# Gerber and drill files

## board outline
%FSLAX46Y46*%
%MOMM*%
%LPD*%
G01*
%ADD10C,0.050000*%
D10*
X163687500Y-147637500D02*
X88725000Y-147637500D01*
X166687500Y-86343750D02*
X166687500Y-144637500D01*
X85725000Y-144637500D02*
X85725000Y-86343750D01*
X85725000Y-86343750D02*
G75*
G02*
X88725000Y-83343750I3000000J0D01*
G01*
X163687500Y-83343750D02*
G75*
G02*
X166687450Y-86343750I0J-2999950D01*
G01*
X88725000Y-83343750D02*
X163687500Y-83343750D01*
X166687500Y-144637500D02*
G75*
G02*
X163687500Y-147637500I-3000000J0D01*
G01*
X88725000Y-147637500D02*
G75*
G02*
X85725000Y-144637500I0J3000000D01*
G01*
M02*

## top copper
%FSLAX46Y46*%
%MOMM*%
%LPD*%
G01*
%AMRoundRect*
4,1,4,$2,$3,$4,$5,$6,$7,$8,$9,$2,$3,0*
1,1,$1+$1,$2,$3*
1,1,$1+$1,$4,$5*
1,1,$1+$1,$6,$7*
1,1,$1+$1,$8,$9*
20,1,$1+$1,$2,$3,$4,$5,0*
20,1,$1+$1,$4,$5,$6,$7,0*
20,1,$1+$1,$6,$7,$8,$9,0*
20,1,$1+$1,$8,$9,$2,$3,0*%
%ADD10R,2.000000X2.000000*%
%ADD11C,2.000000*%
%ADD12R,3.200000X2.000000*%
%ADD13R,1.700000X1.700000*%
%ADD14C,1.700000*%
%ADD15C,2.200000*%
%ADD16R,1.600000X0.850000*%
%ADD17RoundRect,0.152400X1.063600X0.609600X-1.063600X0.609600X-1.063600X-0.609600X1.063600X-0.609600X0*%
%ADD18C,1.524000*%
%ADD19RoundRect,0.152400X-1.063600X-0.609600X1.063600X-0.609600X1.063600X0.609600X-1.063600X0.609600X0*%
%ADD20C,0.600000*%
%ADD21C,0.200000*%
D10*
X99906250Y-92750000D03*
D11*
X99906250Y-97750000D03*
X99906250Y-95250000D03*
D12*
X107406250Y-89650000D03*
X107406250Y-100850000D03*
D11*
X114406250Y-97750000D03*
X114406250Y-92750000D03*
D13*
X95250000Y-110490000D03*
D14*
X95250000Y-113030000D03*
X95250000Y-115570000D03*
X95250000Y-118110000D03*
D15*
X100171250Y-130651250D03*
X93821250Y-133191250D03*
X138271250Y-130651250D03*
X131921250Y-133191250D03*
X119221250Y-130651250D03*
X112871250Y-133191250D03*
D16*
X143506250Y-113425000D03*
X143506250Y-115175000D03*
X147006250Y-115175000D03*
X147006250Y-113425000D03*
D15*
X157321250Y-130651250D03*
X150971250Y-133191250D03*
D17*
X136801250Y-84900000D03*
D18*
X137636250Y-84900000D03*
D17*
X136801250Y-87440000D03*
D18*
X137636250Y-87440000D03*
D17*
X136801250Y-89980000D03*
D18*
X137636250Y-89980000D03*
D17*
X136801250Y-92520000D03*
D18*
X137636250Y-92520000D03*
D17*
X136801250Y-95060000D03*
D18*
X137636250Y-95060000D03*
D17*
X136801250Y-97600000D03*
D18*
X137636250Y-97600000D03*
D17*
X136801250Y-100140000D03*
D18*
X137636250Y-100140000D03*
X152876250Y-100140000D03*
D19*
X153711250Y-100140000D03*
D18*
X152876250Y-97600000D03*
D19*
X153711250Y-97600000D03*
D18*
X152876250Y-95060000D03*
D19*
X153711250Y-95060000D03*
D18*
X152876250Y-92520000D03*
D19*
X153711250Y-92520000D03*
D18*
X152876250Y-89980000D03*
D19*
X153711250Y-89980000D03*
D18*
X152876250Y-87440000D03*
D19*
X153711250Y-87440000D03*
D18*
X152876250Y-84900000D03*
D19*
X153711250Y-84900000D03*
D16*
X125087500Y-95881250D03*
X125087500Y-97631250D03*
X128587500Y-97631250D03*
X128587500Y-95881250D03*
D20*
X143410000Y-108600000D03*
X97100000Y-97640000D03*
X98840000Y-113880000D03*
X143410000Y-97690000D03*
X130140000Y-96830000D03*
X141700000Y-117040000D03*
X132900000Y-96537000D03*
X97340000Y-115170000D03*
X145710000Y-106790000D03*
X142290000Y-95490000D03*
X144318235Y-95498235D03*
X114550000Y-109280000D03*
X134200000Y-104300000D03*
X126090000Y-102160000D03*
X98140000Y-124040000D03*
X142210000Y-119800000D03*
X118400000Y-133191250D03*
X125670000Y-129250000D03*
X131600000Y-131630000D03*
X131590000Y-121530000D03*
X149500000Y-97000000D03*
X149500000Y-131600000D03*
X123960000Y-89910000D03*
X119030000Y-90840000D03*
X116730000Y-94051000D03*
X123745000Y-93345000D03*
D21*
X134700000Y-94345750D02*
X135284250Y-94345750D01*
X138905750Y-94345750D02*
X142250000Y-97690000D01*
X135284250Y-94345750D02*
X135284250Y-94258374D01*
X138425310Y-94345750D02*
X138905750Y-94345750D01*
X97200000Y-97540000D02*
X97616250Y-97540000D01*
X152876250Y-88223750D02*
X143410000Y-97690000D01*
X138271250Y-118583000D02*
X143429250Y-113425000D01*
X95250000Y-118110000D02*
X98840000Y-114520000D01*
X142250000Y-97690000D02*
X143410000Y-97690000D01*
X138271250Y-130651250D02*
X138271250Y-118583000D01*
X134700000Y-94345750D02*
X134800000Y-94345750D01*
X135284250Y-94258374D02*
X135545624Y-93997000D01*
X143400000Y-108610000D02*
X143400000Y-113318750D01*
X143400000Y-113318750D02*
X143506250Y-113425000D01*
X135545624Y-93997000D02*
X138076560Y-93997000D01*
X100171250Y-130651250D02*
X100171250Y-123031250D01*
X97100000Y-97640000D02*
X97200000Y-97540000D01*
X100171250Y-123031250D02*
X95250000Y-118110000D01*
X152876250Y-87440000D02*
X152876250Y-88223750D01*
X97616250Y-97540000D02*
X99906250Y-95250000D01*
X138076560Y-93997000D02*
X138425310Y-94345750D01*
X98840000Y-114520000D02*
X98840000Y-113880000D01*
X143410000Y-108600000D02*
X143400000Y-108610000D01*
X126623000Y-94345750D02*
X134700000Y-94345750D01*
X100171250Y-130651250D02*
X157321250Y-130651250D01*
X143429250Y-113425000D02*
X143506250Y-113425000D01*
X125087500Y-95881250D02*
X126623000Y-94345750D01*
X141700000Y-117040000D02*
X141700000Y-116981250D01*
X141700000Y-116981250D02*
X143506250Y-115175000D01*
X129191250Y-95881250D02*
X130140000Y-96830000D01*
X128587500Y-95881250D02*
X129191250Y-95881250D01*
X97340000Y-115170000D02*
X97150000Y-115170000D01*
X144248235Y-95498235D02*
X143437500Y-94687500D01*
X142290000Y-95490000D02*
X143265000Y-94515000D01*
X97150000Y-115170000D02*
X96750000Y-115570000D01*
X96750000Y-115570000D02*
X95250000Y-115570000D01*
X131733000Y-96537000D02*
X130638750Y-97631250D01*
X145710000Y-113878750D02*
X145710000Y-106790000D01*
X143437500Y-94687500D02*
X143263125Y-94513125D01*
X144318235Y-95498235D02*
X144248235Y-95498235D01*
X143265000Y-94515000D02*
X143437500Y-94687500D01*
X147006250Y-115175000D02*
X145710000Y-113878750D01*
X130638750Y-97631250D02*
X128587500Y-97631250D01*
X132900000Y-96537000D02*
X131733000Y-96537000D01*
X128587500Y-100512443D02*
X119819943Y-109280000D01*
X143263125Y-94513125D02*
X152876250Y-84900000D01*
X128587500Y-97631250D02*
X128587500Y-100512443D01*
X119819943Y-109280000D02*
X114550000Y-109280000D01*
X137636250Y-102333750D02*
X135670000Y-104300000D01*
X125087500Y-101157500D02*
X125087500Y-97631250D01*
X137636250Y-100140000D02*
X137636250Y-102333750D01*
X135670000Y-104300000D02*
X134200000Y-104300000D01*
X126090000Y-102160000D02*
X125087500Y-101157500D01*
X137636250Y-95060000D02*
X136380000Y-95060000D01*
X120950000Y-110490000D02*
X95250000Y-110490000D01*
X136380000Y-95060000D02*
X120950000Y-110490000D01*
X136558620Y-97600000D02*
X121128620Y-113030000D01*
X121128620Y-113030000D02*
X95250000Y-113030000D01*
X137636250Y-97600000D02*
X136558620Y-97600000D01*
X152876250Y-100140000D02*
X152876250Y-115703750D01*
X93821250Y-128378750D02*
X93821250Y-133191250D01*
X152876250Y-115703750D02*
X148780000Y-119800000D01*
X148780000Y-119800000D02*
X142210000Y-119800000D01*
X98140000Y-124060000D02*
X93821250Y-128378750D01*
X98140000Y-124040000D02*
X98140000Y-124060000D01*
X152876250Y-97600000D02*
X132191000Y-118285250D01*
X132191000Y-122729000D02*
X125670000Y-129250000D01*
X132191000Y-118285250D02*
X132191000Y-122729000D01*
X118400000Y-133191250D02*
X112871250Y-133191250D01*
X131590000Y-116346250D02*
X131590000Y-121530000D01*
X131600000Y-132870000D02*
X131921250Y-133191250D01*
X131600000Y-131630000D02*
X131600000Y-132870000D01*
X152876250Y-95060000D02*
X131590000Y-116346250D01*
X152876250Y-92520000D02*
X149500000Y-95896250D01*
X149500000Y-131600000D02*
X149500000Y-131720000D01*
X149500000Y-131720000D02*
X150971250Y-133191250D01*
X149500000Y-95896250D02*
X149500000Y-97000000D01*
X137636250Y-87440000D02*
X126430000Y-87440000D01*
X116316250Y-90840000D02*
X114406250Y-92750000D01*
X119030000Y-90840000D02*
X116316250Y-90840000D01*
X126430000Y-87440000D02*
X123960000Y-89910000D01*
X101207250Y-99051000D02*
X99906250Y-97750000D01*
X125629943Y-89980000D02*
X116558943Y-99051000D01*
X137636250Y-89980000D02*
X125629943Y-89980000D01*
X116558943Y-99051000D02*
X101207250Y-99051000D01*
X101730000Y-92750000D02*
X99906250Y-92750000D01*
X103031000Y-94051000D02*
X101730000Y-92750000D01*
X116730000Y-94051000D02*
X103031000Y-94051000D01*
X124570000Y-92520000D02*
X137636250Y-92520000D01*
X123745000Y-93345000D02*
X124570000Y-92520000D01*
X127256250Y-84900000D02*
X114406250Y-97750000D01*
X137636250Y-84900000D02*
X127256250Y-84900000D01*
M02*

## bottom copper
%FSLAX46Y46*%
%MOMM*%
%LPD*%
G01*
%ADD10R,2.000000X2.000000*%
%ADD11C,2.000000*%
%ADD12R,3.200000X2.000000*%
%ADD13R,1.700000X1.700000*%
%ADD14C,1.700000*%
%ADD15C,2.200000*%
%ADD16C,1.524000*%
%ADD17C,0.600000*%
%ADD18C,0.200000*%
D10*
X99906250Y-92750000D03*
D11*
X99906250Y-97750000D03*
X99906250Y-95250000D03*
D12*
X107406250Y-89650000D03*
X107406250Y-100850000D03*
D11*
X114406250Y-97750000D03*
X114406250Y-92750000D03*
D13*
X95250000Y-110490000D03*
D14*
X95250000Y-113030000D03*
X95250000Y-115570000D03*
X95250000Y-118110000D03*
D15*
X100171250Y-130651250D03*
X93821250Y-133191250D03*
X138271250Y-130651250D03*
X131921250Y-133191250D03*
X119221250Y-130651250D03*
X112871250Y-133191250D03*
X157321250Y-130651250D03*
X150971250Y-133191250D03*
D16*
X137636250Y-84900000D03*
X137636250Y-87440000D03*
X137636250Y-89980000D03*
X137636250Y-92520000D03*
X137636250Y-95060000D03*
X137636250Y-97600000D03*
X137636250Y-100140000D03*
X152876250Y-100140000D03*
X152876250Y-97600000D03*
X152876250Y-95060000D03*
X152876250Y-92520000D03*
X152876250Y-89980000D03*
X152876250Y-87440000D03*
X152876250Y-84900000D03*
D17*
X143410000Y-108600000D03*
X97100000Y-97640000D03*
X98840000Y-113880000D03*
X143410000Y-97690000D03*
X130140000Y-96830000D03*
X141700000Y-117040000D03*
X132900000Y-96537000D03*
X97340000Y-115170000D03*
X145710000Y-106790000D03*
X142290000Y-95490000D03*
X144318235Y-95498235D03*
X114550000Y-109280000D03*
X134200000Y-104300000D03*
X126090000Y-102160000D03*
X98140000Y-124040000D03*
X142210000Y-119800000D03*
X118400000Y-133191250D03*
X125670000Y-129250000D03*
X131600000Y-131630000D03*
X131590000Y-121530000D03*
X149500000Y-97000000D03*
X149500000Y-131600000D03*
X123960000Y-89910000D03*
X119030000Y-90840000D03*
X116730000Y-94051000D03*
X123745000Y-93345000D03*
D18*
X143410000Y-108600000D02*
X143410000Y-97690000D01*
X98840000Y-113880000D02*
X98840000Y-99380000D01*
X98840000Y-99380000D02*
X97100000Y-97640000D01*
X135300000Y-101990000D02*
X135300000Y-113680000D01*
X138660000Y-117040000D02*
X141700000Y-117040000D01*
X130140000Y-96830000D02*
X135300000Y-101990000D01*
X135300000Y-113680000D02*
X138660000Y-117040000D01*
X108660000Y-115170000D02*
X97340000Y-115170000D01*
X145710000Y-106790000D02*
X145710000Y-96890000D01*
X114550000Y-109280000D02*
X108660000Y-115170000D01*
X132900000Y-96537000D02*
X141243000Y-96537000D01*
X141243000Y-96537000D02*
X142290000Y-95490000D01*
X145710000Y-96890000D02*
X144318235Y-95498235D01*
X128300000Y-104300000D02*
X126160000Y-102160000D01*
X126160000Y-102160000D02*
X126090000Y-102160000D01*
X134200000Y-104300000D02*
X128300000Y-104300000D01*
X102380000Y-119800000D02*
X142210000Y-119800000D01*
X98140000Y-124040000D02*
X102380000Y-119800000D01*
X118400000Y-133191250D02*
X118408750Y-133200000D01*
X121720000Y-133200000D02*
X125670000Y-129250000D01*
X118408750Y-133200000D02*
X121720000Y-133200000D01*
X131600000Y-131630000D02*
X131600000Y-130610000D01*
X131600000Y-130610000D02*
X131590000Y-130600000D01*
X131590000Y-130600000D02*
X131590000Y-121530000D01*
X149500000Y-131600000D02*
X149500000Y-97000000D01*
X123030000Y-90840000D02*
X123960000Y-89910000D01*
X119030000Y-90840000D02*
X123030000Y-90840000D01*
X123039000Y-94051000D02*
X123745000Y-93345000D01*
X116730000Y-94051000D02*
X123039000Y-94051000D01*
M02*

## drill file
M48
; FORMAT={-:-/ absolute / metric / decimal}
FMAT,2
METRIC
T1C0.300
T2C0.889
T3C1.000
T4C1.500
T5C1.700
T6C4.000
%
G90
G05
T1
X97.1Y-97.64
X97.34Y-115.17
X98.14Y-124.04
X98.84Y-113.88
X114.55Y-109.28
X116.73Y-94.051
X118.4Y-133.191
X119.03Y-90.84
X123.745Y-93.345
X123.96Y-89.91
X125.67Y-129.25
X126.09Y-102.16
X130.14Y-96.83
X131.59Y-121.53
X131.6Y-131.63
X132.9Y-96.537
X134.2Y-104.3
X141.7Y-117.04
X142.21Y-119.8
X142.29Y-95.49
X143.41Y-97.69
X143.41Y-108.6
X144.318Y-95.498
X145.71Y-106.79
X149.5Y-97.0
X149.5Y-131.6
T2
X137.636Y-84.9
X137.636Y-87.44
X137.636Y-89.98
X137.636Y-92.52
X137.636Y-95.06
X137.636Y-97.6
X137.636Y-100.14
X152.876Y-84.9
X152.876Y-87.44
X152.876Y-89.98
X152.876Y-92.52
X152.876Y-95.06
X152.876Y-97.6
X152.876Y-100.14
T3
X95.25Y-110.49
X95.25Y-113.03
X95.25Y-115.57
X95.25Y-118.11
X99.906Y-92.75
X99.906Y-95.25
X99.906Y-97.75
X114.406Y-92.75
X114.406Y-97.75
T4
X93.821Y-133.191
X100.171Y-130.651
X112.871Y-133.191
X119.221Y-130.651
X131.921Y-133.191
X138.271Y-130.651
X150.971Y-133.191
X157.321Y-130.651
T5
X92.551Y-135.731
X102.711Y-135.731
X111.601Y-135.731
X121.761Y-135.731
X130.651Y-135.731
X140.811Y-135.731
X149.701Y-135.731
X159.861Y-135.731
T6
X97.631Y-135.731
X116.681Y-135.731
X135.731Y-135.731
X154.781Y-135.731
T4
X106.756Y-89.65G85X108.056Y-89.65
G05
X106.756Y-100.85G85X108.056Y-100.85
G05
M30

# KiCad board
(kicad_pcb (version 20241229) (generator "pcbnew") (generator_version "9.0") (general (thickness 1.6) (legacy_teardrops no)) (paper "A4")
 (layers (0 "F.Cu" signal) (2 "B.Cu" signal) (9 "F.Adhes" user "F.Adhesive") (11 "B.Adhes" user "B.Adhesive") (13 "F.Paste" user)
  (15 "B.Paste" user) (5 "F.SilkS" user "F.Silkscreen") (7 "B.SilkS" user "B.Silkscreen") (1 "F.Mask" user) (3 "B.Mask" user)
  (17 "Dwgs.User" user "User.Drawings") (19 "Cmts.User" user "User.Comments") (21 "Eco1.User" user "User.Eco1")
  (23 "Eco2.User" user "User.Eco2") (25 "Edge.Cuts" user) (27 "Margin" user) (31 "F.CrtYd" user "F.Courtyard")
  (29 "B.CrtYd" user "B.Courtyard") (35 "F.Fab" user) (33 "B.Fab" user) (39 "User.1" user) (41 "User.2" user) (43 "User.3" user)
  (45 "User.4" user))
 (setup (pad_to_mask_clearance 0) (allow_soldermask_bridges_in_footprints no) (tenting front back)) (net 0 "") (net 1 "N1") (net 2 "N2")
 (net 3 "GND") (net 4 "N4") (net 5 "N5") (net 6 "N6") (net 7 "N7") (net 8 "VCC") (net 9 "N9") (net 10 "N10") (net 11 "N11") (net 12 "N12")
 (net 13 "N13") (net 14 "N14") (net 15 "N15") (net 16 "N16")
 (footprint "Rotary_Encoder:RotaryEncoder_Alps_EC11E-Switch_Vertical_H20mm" (layer "F.Cu") (at 99.90625 92.75)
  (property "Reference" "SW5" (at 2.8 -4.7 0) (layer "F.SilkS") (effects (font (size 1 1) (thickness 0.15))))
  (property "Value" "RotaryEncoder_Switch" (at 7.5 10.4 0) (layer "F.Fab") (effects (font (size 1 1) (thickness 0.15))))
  (pad "A" thru_hole rect (at 0 0) (size 2 2) (drill 1) (layers "*.Cu" "*.Mask") (remove_unused_layers no) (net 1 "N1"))
  (pad "B" thru_hole circle (at 0 5) (size 2 2) (drill 1) (layers "*.Cu" "*.Mask") (remove_unused_layers no) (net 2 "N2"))
  (pad "C" thru_hole circle (at 0 2.5) (size 2 2) (drill 1) (layers "*.Cu" "*.Mask") (remove_unused_layers no) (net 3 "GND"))
  (pad "MP" thru_hole rect (at 7.5 -3.1) (size 3.2 2) (drill oval 2.8 1.5) (layers "*.Cu" "*.Mask") (remove_unused_layers no))
  (pad "MP" thru_hole rect (at 7.5 8.1) (size 3.2 2) (drill oval 2.8 1.5) (layers "*.Cu" "*.Mask") (remove_unused_layers no))
  (pad "S1" thru_hole circle (at 14.5 5) (size 2 2) (drill 1) (layers "*.Cu" "*.Mask") (remove_unused_layers no) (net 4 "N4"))
  (pad "S2" thru_hole circle (at 14.5 0) (size 2 2) (drill 1) (layers "*.Cu" "*.Mask") (remove_unused_layers no) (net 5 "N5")))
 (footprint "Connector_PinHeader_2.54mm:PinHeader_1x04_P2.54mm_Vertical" (layer "F.Cu") (at 95.25 110.49)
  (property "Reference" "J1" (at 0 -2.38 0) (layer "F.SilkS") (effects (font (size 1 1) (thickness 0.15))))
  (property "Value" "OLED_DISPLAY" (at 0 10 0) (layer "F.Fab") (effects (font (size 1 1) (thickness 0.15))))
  (pad "1" thru_hole rect (at 0 0) (size 1.7 1.7) (drill 1) (layers "*.Cu" "*.Mask") (remove_unused_layers no) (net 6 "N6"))
  (pad "2" thru_hole circle (at 0 2.54) (size 1.7 1.7) (drill 1) (layers "*.Cu" "*.Mask") (remove_unused_layers no) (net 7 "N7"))
  (pad "3" thru_hole circle (at 0 5.08) (size 1.7 1.7) (drill 1) (layers "*.Cu" "*.Mask") (remove_unused_layers no) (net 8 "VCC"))
  (pad "4" thru_hole circle (at 0 7.62) (size 1.7 1.7) (drill 1) (layers "*.Cu" "*.Mask") (remove_unused_layers no) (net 3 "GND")))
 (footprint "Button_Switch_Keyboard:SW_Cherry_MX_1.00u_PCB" (layer "F.Cu") (at 100.17125 130.65125)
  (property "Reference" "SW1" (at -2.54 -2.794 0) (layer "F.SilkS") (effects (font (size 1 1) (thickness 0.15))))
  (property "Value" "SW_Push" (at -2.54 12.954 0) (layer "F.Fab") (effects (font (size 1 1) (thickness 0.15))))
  (pad "" np_thru_hole circle (at -7.62 5.08) (size 1.7 1.7) (drill 1.7) (layers "*.Cu" "*.Mask"))
  (pad "" np_thru_hole circle (at -2.54 5.08) (size 4 4) (drill 4) (layers "*.Cu" "*.Mask"))
  (pad "" np_thru_hole circle (at 2.54 5.08) (size 1.7 1.7) (drill 1.7) (layers "*.Cu" "*.Mask"))
  (pad "1" thru_hole circle (at 0 0) (size 2.2 2.2) (drill 1.5) (layers "*.Cu" "*.Mask") (remove_unused_layers no) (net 3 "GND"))
  (pad "2" thru_hole circle (at -6.35 2.54) (size 2.2 2.2) (drill 1.5) (layers "*.Cu" "*.Mask") (remove_unused_layers no) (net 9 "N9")))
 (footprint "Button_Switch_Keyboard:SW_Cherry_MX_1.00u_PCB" (layer "F.Cu") (at 138.27125 130.65125)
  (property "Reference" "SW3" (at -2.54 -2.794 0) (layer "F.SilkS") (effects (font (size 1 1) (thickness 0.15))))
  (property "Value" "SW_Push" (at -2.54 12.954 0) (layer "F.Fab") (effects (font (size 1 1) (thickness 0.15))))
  (pad "" np_thru_hole circle (at -7.62 5.08) (size 1.7 1.7) (drill 1.7) (layers "*.Cu" "*.Mask"))
  (pad "" np_thru_hole circle (at -2.54 5.08) (size 4 4) (drill 4) (layers "*.Cu" "*.Mask"))
  (pad "" np_thru_hole circle (at 2.54 5.08) (size 1.7 1.7) (drill 1.7) (layers "*.Cu" "*.Mask"))
  (pad "1" thru_hole circle (at 0 0) (size 2.2 2.2) (drill 1.5) (layers "*.Cu" "*.Mask") (remove_unused_layers no) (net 3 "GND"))
  (pad "2" thru_hole circle (at -6.35 2.54) (size 2.2 2.2) (drill 1.5) (layers "*.Cu" "*.Mask") (remove_unused_layers no) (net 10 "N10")))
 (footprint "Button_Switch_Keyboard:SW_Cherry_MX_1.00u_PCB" (layer "F.Cu") (at 119.22125 130.65125)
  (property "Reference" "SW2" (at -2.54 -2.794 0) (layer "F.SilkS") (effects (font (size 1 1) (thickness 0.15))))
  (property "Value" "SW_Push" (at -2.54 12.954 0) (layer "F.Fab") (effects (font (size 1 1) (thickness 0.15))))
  (pad "" np_thru_hole circle (at -7.62 5.08) (size 1.7 1.7) (drill 1.7) (layers "*.Cu" "*.Mask"))
  (pad "" np_thru_hole circle (at -2.54 5.08) (size 4 4) (drill 4) (layers "*.Cu" "*.Mask"))
  (pad "" np_thru_hole circle (at 2.54 5.08) (size 1.7 1.7) (drill 1.7) (layers "*.Cu" "*.Mask"))
  (pad "1" thru_hole circle (at 0 0) (size 2.2 2.2) (drill 1.5) (layers "*.Cu" "*.Mask") (remove_unused_layers no) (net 3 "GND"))
  (pad "2" thru_hole circle (at -6.35 2.54) (size 2.2 2.2) (drill 1.5) (layers "*.Cu" "*.Mask") (remove_unused_layers no) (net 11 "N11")))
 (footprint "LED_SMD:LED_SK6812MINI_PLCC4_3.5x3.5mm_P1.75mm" (layer "F.Cu") (at 145.25625 114.3)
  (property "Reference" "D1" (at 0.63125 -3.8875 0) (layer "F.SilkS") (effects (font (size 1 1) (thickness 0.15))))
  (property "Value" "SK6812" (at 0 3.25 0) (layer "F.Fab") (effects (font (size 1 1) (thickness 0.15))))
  (pad "1" smd rect (at -1.75 -0.875) (size 1.6 0.85) (layers "F.Cu" "F.Mask" "F.Paste") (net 3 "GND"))
  (pad "2" smd rect (at -1.75 0.875) (size 1.6 0.85) (layers "F.Cu" "F.Mask" "F.Paste") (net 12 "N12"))
  (pad "3" smd rect (at 1.75 0.875) (size 1.6 0.85) (layers "F.Cu" "F.Mask" "F.Paste") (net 8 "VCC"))
  (pad "4" smd rect (at 1.75 -0.875) (size 1.6 0.85) (layers "F.Cu" "F.Mask" "F.Paste") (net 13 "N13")))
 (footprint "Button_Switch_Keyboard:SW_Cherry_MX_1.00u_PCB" (layer "F.Cu") (at 157.32125 130.65125)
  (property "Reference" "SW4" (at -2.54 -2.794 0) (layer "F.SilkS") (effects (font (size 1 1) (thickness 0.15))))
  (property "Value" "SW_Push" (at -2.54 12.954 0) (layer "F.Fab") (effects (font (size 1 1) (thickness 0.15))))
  (pad "" np_thru_hole circle (at -7.62 5.08) (size 1.7 1.7) (drill 1.7) (layers "*.Cu" "*.Mask"))
  (pad "" np_thru_hole circle (at -2.54 5.08) (size 4 4) (drill 4) (layers "*.Cu" "*.Mask"))
  (pad "" np_thru_hole circle (at 2.54 5.08) (size 1.7 1.7) (drill 1.7) (layers "*.Cu" "*.Mask"))
  (pad "1" thru_hole circle (at 0 0) (size 2.2 2.2) (drill 1.5) (layers "*.Cu" "*.Mask") (remove_unused_layers no) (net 3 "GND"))
  (pad "2" thru_hole circle (at -6.35 2.54) (size 2.2 2.2) (drill 1.5) (layers "*.Cu" "*.Mask") (remove_unused_layers no) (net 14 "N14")))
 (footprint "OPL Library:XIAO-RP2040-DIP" (layer "F.Cu") (at 145.25625 92.52)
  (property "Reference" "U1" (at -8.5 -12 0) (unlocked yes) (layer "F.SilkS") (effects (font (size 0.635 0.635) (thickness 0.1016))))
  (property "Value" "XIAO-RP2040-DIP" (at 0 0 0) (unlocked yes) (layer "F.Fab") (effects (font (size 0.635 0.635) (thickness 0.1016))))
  (pad "1" smd roundrect (at -8.455 -7.62 180) (size 2.432 1.524) (layers "F.Cu" "F.Mask") (roundrect_rratio 0.1) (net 4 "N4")
   (thermal_bridge_angle 45))
  (pad "1" thru_hole circle (at -7.62 -7.62 180) (size 1.524 1.524) (drill 0.889) (layers "*.Cu" "*.Mask") (remove_unused_layers no)
   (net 4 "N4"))
  (pad "2" smd roundrect (at -8.455 -5.08 180) (size 2.432 1.524) (layers "F.Cu" "F.Mask") (roundrect_rratio 0.1) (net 5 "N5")
   (thermal_bridge_angle 45))
  (pad "2" thru_hole circle (at -7.62 -5.08 180) (size 1.524 1.524) (drill 0.889) (layers "*.Cu" "*.Mask") (remove_unused_layers no)
   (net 5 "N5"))
  (pad "3" smd roundrect (at -8.455 -2.54 180) (size 2.432 1.524) (layers "F.Cu" "F.Mask") (roundrect_rratio 0.1) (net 2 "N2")
   (thermal_bridge_angle 45))
  (pad "3" thru_hole circle (at -7.62 -2.54 180) (size 1.524 1.524) (drill 0.889) (layers "*.Cu" "*.Mask") (remove_unused_layers no)
   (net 2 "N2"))
  (pad "4" smd roundrect (at -8.455 0 180) (size 2.432 1.524) (layers "F.Cu" "F.Mask") (roundrect_rratio 0.1) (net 1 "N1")
   (thermal_bridge_angle 45))
  (pad "4" thru_hole circle (at -7.62 0 180) (size 1.524 1.524) (drill 0.889) (layers "*.Cu" "*.Mask") (remove_unused_layers no)
   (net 1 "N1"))
  (pad "5" smd roundrect (at -8.455 2.54 180) (size 2.432 1.524) (layers "F.Cu" "F.Mask") (roundrect_rratio 0.1) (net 6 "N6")
   (thermal_bridge_angle 45))
  (pad "5" thru_hole circle (at -7.62 2.54 180) (size 1.524 1.524) (drill 0.889) (layers "*.Cu" "*.Mask") (remove_unused_layers no)
   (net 6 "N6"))
  (pad "6" smd roundrect (at -8.455 5.08 180) (size 2.432 1.524) (layers "F.Cu" "F.Mask") (roundrect_rratio 0.1) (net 7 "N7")
   (thermal_bridge_angle 45))
  (pad "6" thru_hole circle (at -7.62 5.08 180) (size 1.524 1.524) (drill 0.889) (layers "*.Cu" "*.Mask") (remove_unused_layers no)
   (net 7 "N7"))
  (pad "7" smd roundrect (at -8.455 7.62 180) (size 2.432 1.524) (layers "F.Cu" "F.Mask") (roundrect_rratio 0.1) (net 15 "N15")
   (thermal_bridge_angle 45))
  (pad "7" thru_hole circle (at -7.62 7.62 180) (size 1.524 1.524) (drill 0.889) (layers "*.Cu" "*.Mask") (remove_unused_layers no)
   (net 15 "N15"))
  (pad "8" thru_hole circle (at 7.62 7.62) (size 1.524 1.524) (drill 0.889) (layers "*.Cu" "*.Mask") (remove_unused_layers no) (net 9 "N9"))
  (pad "8" smd roundrect (at 8.455 7.62) (size 2.432 1.524) (layers "F.Cu" "F.Mask") (roundrect_rratio 0.1) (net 9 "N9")
   (thermal_bridge_angle 45))
  (pad "9" thru_hole circle (at 7.62 5.08) (size 1.524 1.524) (drill 0.889) (layers "*.Cu" "*.Mask") (remove_unused_layers no)
   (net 11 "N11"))
  (pad "9" smd roundrect (at 8.455 5.08) (size 2.432 1.524) (layers "F.Cu" "F.Mask") (roundrect_rratio 0.1) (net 11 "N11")
   (thermal_bridge_angle 45))
  (pad "10" thru_hole circle (at 7.62 2.54) (size 1.524 1.524) (drill 0.889) (layers "*.Cu" "*.Mask") (remove_unused_layers no)
   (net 10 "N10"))
  (pad "10" smd roundrect (at 8.455 2.54) (size 2.432 1.524) (layers "F.Cu" "F.Mask") (roundrect_rratio 0.1) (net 10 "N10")
   (thermal_bridge_angle 45))
  (pad "11" thru_hole circle (at 7.62 0) (size 1.524 1.524) (drill 0.889) (layers "*.Cu" "*.Mask") (remove_unused_layers no) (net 14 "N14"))
  (pad "11" smd roundrect (at 8.455 0) (size 2.432 1.524) (layers "F.Cu" "F.Mask") (roundrect_rratio 0.1) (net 14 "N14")
   (thermal_bridge_angle 45))
  (pad "12" thru_hole circle (at 7.62 -2.54) (size 1.524 1.524) (drill 0.889) (layers "*.Cu" "*.Mask") (remove_unused_layers no)
   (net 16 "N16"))
  (pad "12" smd roundrect (at 8.455 -2.54) (size 2.432 1.524) (layers "F.Cu" "F.Mask") (roundrect_rratio 0.1) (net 16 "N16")
   (thermal_bridge_angle 45))
  (pad "13" thru_hole circle (at 7.62 -5.08) (size 1.524 1.524) (drill 0.889) (layers "*.Cu" "*.Mask") (remove_unused_layers no)
   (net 3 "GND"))
  (pad "13" smd roundrect (at 8.455 -5.08) (size 2.432 1.524) (layers "F.Cu" "F.Mask") (roundrect_rratio 0.1) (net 3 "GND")
   (thermal_bridge_angle 45))
  (pad "14" thru_hole circle (at 7.62 -7.62) (size 1.524 1.524) (drill 0.889) (layers "*.Cu" "*.Mask") (remove_unused_layers no)
   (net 8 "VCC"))
  (pad "14" smd roundrect (at 8.455 -7.62) (size 2.432 1.524) (layers "F.Cu" "F.Mask") (roundrect_rratio 0.1) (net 8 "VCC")
   (thermal_bridge_angle 45)))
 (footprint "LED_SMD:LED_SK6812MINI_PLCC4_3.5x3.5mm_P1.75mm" (layer "F.Cu") (at 126.8375 96.75625)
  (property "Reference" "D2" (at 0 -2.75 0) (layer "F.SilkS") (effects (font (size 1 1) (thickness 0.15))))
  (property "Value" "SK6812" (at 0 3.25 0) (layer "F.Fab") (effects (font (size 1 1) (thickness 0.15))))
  (pad "1" smd rect (at -1.75 -0.875) (size 1.6 0.85) (layers "F.Cu" "F.Mask" "F.Paste") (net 3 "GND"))
  (pad "2" smd rect (at -1.75 0.875) (size 1.6 0.85) (layers "F.Cu" "F.Mask" "F.Paste") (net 15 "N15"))
  (pad "3" smd rect (at 1.75 0.875) (size 1.6 0.85) (layers "F.Cu" "F.Mask" "F.Paste") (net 8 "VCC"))
  (pad "4" smd rect (at 1.75 -0.875) (size 1.6 0.85) (layers "F.Cu" "F.Mask" "F.Paste") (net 12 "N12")))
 (gr_line (start 163.6875 147.6375) (end 88.725 147.6375) (stroke (width 0.05) (type default)) (layer "Edge.Cuts"))
 (gr_line (start 166.6875 86.34375) (end 166.6875 144.6375) (stroke (width 0.05) (type default)) (layer "Edge.Cuts"))
 (gr_line (start 85.725 144.6375) (end 85.725 86.34375) (stroke (width 0.05) (type default)) (layer "Edge.Cuts"))
 (gr_arc (start 85.725 86.34375) (mid 86.60368 84.22243) (end 88.725 83.34375) (stroke (width 0.05) (type default)) (layer "Edge.Cuts"))
 (gr_arc (start 163.6875 83.34375) (mid 165.808838 84.222427) (end 166.6875 86.34375) (stroke (width 0.05) (type default))
  (layer "Edge.Cuts"))
 (gr_line (start 88.725 83.34375) (end 163.6875 83.34375) (stroke (width 0.05) (type default)) (layer "Edge.Cuts"))
 (gr_arc (start 166.6875 144.6375) (mid 165.80882 146.75882) (end 163.6875 147.6375) (stroke (width 0.05) (type default))
  (layer "Edge.Cuts"))
 (gr_arc (start 88.725 147.6375) (mid 86.60368 146.75882) (end 85.725 144.6375) (stroke (width 0.05) (type default)) (layer "Edge.Cuts"))
 (segment (start 134.7 94.34575) (end 135.28425 94.34575) (width 0.2) (layer "F.Cu") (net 3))
 (segment (start 138.90575 94.34575) (end 142.25 97.69) (width 0.2) (layer "F.Cu") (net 3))
 (segment (start 135.28425 94.34575) (end 135.28425 94.258374) (width 0.2) (layer "F.Cu") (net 3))
 (segment (start 138.42531 94.34575) (end 138.90575 94.34575) (width 0.2) (layer "F.Cu") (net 3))
 (segment (start 97.2 97.54) (end 97.61625 97.54) (width 0.2) (layer "F.Cu") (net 3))
 (segment (start 152.87625 88.22375) (end 143.41 97.69) (width 0.2) (layer "F.Cu") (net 3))
 (segment (start 138.27125 118.583) (end 143.42925 113.425) (width 0.2) (layer "F.Cu") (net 3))
 (segment (start 95.25 118.11) (end 98.84 114.52) (width 0.2) (layer "F.Cu") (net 3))
 (segment (start 142.25 97.69) (end 143.41 97.69) (width 0.2) (layer "F.Cu") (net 3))
 (segment (start 138.27125 130.65125) (end 138.27125 118.583) (width 0.2) (layer "F.Cu") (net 3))
 (segment (start 134.7 94.34575) (end 134.8 94.34575) (width 0.2) (layer "F.Cu") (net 3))
 (segment (start 135.28425 94.258374) (end 135.545624 93.997) (width 0.2) (layer "F.Cu") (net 3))
 (segment (start 143.4 108.61) (end 143.4 113.31875) (width 0.2) (layer "F.Cu") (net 3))
 (segment (start 143.4 113.31875) (end 143.50625 113.425) (width 0.2) (layer "F.Cu") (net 3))
 (segment (start 135.545624 93.997) (end 138.07656 93.997) (width 0.2) (layer "F.Cu") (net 3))
 (segment (start 100.17125 130.65125) (end 100.17125 123.03125) (width 0.2) (layer "F.Cu") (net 3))
 (segment (start 97.1 97.64) (end 97.2 97.54) (width 0.2) (layer "F.Cu") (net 3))
 (segment (start 100.17125 123.03125) (end 95.25 118.11) (width 0.2) (layer "F.Cu") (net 3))
 (segment (start 152.87625 87.44) (end 152.87625 88.22375) (width 0.2) (layer "F.Cu") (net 3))
 (segment (start 97.61625 97.54) (end 99.90625 95.25) (width 0.2) (layer "F.Cu") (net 3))
 (segment (start 138.07656 93.997) (end 138.42531 94.34575) (width 0.2) (layer "F.Cu") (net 3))
 (segment (start 98.84 114.52) (end 98.84 113.88) (width 0.2) (layer "F.Cu") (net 3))
 (segment (start 143.41 108.6) (end 143.4 108.61) (width 0.2) (layer "F.Cu") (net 3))
 (segment (start 126.623 94.34575) (end 134.7 94.34575) (width 0.2) (layer "F.Cu") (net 3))
 (segment (start 100.17125 130.65125) (end 157.32125 130.65125) (width 0.2) (layer "F.Cu") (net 3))
 (segment (start 143.42925 113.425) (end 143.50625 113.425) (width 0.2) (layer "F.Cu") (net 3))
 (segment (start 125.0875 95.88125) (end 126.623 94.34575) (width 0.2) (layer "F.Cu") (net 3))
 (via (at 143.41 108.6) (size 0.6) (drill 0.3) (layers "F.Cu" "B.Cu") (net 3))
 (via (at 97.1 97.64) (size 0.6) (drill 0.3) (layers "F.Cu" "B.Cu") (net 3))
 (via (at 98.84 113.88) (size 0.6) (drill 0.3) (layers "F.Cu" "B.Cu") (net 3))
 (via (at 143.41 97.69) (size 0.6) (drill 0.3) (layers "F.Cu" "B.Cu") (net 3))
 (segment (start 143.41 108.6) (end 143.41 97.69) (width 0.2) (layer "B.Cu") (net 3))
 (segment (start 98.84 113.88) (end 98.84 99.38) (width 0.2) (layer "B.Cu") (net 3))
 (segment (start 98.84 99.38) (end 97.1 97.64) (width 0.2) (layer "B.Cu") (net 3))
 (segment (start 141.7 117.04) (end 141.7 116.98125) (width 0.2) (layer "F.Cu") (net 12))
 (segment (start 141.7 116.98125) (end 143.50625 115.175) (width 0.2) (layer "F.Cu") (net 12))
 (segment (start 129.19125 95.88125) (end 130.14 96.83) (width 0.2) (layer "F.Cu") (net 12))
 (segment (start 128.5875 95.88125) (end 129.19125 95.88125) (width 0.2) (layer "F.Cu") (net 12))
 (via (at 130.14 96.83) (size 0.6) (drill 0.3) (layers "F.Cu" "B.Cu") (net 12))
 (via (at 141.7 117.04) (size 0.6) (drill 0.3) (layers "F.Cu" "B.Cu") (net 12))
 (segment (start 135.3 101.99) (end 135.3 113.68) (width 0.2) (layer "B.Cu") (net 12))
 (segment (start 138.66 117.04) (end 141.7 117.04) (width 0.2) (layer "B.Cu") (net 12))
 (segment (start 130.14 96.83) (end 135.3 101.99) (width 0.2) (layer "B.Cu") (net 12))
 (segment (start 135.3 113.68) (end 138.66 117.04) (width 0.2) (layer "B.Cu") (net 12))
 (segment (start 97.34 115.17) (end 97.15 115.17) (width 0.2) (layer "F.Cu") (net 8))
 (segment (start 144.248235 95.498235) (end 143.4375 94.6875) (width 0.2) (layer "F.Cu") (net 8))
 (segment (start 142.29 95.49) (end 143.265 94.515) (width 0.2) (layer "F.Cu") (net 8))
 (segment (start 97.15 115.17) (end 96.75 115.57) (width 0.2) (layer "F.Cu") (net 8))
 (segment (start 96.75 115.57) (end 95.25 115.57) (width 0.2) (layer "F.Cu") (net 8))
 (segment (start 131.733 96.537) (end 130.63875 97.63125) (width 0.2) (layer "F.Cu") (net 8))
 (segment (start 145.71 113.87875) (end 145.71 106.79) (width 0.2) (layer "F.Cu") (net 8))
 (segment (start 143.4375 94.6875) (end 143.263125 94.513125) (width 0.2) (layer "F.Cu") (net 8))
 (segment (start 144.318235 95.498235) (end 144.248235 95.498235) (width 0.2) (layer "F.Cu") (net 8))
 (segment (start 143.265 94.515) (end 143.4375 94.6875) (width 0.2) (layer "F.Cu") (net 8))
 (segment (start 147.00625 115.175) (end 145.71 113.87875) (width 0.2) (layer "F.Cu") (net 8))
 (segment (start 130.63875 97.63125) (end 128.5875 97.63125) (width 0.2) (layer "F.Cu") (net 8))
 (segment (start 132.9 96.537) (end 131.733 96.537) (width 0.2) (layer "F.Cu") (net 8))
 (segment (start 128.5875 100.512443) (end 119.819943 109.28) (width 0.2) (layer "F.Cu") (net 8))
 (segment (start 143.263125 94.513125) (end 152.87625 84.9) (width 0.2) (layer "F.Cu") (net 8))
 (segment (start 128.5875 97.63125) (end 128.5875 100.512443) (width 0.2) (layer "F.Cu") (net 8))
 (segment (start 119.819943 109.28) (end 114.55 109.28) (width 0.2) (layer "F.Cu") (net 8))
 (via (at 132.9 96.537) (size 0.6) (drill 0.3) (layers "F.Cu" "B.Cu") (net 8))
 (via (at 97.34 115.17) (size 0.6) (drill 0.3) (layers "F.Cu" "B.Cu") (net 8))
 (via (at 145.71 106.79) (size 0.6) (drill 0.3) (layers "F.Cu" "B.Cu") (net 8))
 (via (at 142.29 95.49) (size 0.6) (drill 0.3) (layers "F.Cu" "B.Cu") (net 8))
 (via (at 144.318235 95.498235) (size 0.6) (drill 0.3) (layers "F.Cu" "B.Cu") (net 8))
 (via (at 114.55 109.28) (size 0.6) (drill 0.3) (layers "F.Cu" "B.Cu") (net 8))
 (segment (start 108.66 115.17) (end 97.34 115.17) (width 0.2) (layer "B.Cu") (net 8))
 (segment (start 145.71 106.79) (end 145.71 96.89) (width 0.2) (layer "B.Cu") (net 8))
 (segment (start 114.55 109.28) (end 108.66 115.17) (width 0.2) (layer "B.Cu") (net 8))
 (segment (start 132.9 96.537) (end 141.243 96.537) (width 0.2) (layer "B.Cu") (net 8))
 (segment (start 141.243 96.537) (end 142.29 95.49) (width 0.2) (layer "B.Cu") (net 8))
 (segment (start 145.71 96.89) (end 144.318235 95.498235) (width 0.2) (layer "B.Cu") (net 8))
 (segment (start 137.63625 102.33375) (end 135.67 104.3) (width 0.2) (layer "F.Cu") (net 15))
 (segment (start 125.0875 101.1575) (end 125.0875 97.63125) (width 0.2) (layer "F.Cu") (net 15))
 (segment (start 137.63625 100.14) (end 137.63625 102.33375) (width 0.2) (layer "F.Cu") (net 15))
 (segment (start 135.67 104.3) (end 134.2 104.3) (width 0.2) (layer "F.Cu") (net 15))
 (segment (start 126.09 102.16) (end 125.0875 101.1575) (width 0.2) (layer "F.Cu") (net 15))
 (via (at 134.2 104.3) (size 0.6) (drill 0.3) (layers "F.Cu" "B.Cu") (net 15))
 (via (at 126.09 102.16) (size 0.6) (drill 0.3) (layers "F.Cu" "B.Cu") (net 15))
 (segment (start 128.3 104.3) (end 126.16 102.16) (width 0.2) (layer "B.Cu") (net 15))
 (segment (start 126.16 102.16) (end 126.09 102.16) (width 0.2) (layer "B.Cu") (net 15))
 (segment (start 134.2 104.3) (end 128.3 104.3) (width 0.2) (layer "B.Cu") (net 15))
 (segment (start 137.63625 95.06) (end 136.38 95.06) (width 0.2) (layer "F.Cu") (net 6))
 (segment (start 120.95 110.49) (end 95.25 110.49) (width 0.2) (layer "F.Cu") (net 6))
 (segment (start 136.38 95.06) (end 120.95 110.49) (width 0.2) (layer "F.Cu") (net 6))
 (segment (start 136.55862 97.6) (end 121.12862 113.03) (width 0.2) (layer "F.Cu") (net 7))
 (segment (start 121.12862 113.03) (end 95.25 113.03) (width 0.2) (layer "F.Cu") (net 7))
 (segment (start 137.63625 97.6) (end 136.55862 97.6) (width 0.2) (layer "F.Cu") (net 7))
 (segment (start 152.87625 100.14) (end 152.87625 115.70375) (width 0.2) (layer "F.Cu") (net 9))
 (segment (start 93.82125 128.37875) (end 93.82125 133.19125) (width 0.2) (layer "F.Cu") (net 9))
 (segment (start 152.87625 115.70375) (end 148.78 119.8) (width 0.2) (layer "F.Cu") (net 9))
 (segment (start 148.78 119.8) (end 142.21 119.8) (width 0.2) (layer "F.Cu") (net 9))
 (segment (start 98.14 124.06) (end 93.82125 128.37875) (width 0.2) (layer "F.Cu") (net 9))
 (segment (start 98.14 124.04) (end 98.14 124.06) (width 0.2) (layer "F.Cu") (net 9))
 (via (at 98.14 124.04) (size 0.6) (drill 0.3) (layers "F.Cu" "B.Cu") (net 9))
 (via (at 142.21 119.8) (size 0.6) (drill 0.3) (layers "F.Cu" "B.Cu") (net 9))
 (segment (start 102.38 119.8) (end 142.21 119.8) (width 0.2) (layer "B.Cu") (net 9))
 (segment (start 98.14 124.04) (end 102.38 119.8) (width 0.2) (layer "B.Cu") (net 9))
 (segment (start 152.87625 97.6) (end 132.191 118.28525) (width 0.2) (layer "F.Cu") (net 11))
 (segment (start 132.191 122.729) (end 125.67 129.25) (width 0.2) (layer "F.Cu") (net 11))
 (segment (start 132.191 118.28525) (end 132.191 122.729) (width 0.2) (layer "F.Cu") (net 11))
 (segment (start 118.4 133.19125) (end 112.87125 133.19125) (width 0.2) (layer "F.Cu") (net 11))
 (via (at 118.4 133.19125) (size 0.6) (drill 0.3) (layers "F.Cu" "B.Cu") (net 11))
 (via (at 125.67 129.25) (size 0.6) (drill 0.3) (layers "F.Cu" "B.Cu") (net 11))
 (segment (start 118.4 133.19125) (end 118.40875 133.2) (width 0.2) (layer "B.Cu") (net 11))
 (segment (start 121.72 133.2) (end 125.67 129.25) (width 0.2) (layer "B.Cu") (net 11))
 (segment (start 118.40875 133.2) (end 121.72 133.2) (width 0.2) (layer "B.Cu") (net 11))
 (segment (start 131.59 116.34625) (end 131.59 121.53) (width 0.2) (layer "F.Cu") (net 10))
 (segment (start 131.6 132.87) (end 131.92125 133.19125) (width 0.2) (layer "F.Cu") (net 10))
 (segment (start 131.6 131.63) (end 131.6 132.87) (width 0.2) (layer "F.Cu") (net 10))
 (segment (start 152.87625 95.06) (end 131.59 116.34625) (width 0.2) (layer "F.Cu") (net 10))
 (via (at 131.6 131.63) (size 0.6) (drill 0.3) (layers "F.Cu" "B.Cu") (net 10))
 (via (at 131.59 121.53) (size 0.6) (drill 0.3) (layers "F.Cu" "B.Cu") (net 10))
 (segment (start 131.6 131.63) (end 131.6 130.61) (width 0.2) (layer "B.Cu") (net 10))
 (segment (start 131.6 130.61) (end 131.59 130.6) (width 0.2) (layer "B.Cu") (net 10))
 (segment (start 131.59 130.6) (end 131.59 121.53) (width 0.2) (layer "B.Cu") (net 10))
 (segment (start 152.87625 92.52) (end 149.5 95.89625) (width 0.2) (layer "F.Cu") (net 14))
 (segment (start 149.5 131.6) (end 149.5 131.72) (width 0.2) (layer "F.Cu") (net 14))
 (segment (start 149.5 131.72) (end 150.97125 133.19125) (width 0.2) (layer "F.Cu") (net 14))
 (segment (start 149.5 95.89625) (end 149.5 97) (width 0.2) (layer "F.Cu") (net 14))
 (via (at 149.5 97) (size 0.6) (drill 0.3) (layers "F.Cu" "B.Cu") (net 14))
 (via (at 149.5 131.6) (size 0.6) (drill 0.3) (layers "F.Cu" "B.Cu") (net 14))
 (segment (start 149.5 131.6) (end 149.5 97) (width 0.2) (layer "B.Cu") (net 14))
 (segment (start 137.63625 87.44) (end 126.43 87.44) (width 0.2) (layer "F.Cu") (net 5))
 (segment (start 116.31625 90.84) (end 114.40625 92.75) (width 0.2) (layer "F.Cu") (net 5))
 (segment (start 119.03 90.84) (end 116.31625 90.84) (width 0.2) (layer "F.Cu") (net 5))
 (segment (start 126.43 87.44) (end 123.96 89.91) (width 0.2) (layer "F.Cu") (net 5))
 (via (at 123.96 89.91) (size 0.6) (drill 0.3) (layers "F.Cu" "B.Cu") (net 5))
 (via (at 119.03 90.84) (size 0.6) (drill 0.3) (layers "F.Cu" "B.Cu") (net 5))
 (segment (start 123.03 90.84) (end 123.96 89.91) (width 0.2) (layer "B.Cu") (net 5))
 (segment (start 119.03 90.84) (end 123.03 90.84) (width 0.2) (layer "B.Cu") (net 5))
 (segment (start 101.20725 99.051) (end 99.90625 97.75) (width 0.2) (layer "F.Cu") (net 2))
 (segment (start 125.629943 89.98) (end 116.558943 99.051) (width 0.2) (layer "F.Cu") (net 2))
 (segment (start 137.63625 89.98) (end 125.629943 89.98) (width 0.2) (layer "F.Cu") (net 2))
 (segment (start 116.558943 99.051) (end 101.20725 99.051) (width 0.2) (layer "F.Cu") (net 2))
 (segment (start 101.73 92.75) (end 99.90625 92.75) (width 0.2) (layer "F.Cu") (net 1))
 (segment (start 103.031 94.051) (end 101.73 92.75) (width 0.2) (layer "F.Cu") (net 1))
 (segment (start 116.73 94.051) (end 103.031 94.051) (width 0.2) (layer "F.Cu") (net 1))
 (segment (start 124.57 92.52) (end 137.63625 92.52) (width 0.2) (layer "F.Cu") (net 1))
 (segment (start 123.745 93.345) (end 124.57 92.52) (width 0.2) (layer "F.Cu") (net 1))
 (via (at 116.73 94.051) (size 0.6) (drill 0.3) (layers "F.Cu" "B.Cu") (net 1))
 (via (at 123.745 93.345) (size 0.6) (drill 0.3) (layers "F.Cu" "B.Cu") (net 1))
 (segment (start 123.039 94.051) (end 123.745 93.345) (width 0.2) (layer "B.Cu") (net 1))
 (segment (start 116.73 94.051) (end 123.039 94.051) (width 0.2) (layer "B.Cu") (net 1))
 (segment (start 127.25625 84.9) (end 114.40625 97.75) (width 0.2) (layer "F.Cu") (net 4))
 (segment (start 137.63625 84.9) (end 127.25625 84.9) (width 0.2) (layer "F.Cu") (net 4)))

